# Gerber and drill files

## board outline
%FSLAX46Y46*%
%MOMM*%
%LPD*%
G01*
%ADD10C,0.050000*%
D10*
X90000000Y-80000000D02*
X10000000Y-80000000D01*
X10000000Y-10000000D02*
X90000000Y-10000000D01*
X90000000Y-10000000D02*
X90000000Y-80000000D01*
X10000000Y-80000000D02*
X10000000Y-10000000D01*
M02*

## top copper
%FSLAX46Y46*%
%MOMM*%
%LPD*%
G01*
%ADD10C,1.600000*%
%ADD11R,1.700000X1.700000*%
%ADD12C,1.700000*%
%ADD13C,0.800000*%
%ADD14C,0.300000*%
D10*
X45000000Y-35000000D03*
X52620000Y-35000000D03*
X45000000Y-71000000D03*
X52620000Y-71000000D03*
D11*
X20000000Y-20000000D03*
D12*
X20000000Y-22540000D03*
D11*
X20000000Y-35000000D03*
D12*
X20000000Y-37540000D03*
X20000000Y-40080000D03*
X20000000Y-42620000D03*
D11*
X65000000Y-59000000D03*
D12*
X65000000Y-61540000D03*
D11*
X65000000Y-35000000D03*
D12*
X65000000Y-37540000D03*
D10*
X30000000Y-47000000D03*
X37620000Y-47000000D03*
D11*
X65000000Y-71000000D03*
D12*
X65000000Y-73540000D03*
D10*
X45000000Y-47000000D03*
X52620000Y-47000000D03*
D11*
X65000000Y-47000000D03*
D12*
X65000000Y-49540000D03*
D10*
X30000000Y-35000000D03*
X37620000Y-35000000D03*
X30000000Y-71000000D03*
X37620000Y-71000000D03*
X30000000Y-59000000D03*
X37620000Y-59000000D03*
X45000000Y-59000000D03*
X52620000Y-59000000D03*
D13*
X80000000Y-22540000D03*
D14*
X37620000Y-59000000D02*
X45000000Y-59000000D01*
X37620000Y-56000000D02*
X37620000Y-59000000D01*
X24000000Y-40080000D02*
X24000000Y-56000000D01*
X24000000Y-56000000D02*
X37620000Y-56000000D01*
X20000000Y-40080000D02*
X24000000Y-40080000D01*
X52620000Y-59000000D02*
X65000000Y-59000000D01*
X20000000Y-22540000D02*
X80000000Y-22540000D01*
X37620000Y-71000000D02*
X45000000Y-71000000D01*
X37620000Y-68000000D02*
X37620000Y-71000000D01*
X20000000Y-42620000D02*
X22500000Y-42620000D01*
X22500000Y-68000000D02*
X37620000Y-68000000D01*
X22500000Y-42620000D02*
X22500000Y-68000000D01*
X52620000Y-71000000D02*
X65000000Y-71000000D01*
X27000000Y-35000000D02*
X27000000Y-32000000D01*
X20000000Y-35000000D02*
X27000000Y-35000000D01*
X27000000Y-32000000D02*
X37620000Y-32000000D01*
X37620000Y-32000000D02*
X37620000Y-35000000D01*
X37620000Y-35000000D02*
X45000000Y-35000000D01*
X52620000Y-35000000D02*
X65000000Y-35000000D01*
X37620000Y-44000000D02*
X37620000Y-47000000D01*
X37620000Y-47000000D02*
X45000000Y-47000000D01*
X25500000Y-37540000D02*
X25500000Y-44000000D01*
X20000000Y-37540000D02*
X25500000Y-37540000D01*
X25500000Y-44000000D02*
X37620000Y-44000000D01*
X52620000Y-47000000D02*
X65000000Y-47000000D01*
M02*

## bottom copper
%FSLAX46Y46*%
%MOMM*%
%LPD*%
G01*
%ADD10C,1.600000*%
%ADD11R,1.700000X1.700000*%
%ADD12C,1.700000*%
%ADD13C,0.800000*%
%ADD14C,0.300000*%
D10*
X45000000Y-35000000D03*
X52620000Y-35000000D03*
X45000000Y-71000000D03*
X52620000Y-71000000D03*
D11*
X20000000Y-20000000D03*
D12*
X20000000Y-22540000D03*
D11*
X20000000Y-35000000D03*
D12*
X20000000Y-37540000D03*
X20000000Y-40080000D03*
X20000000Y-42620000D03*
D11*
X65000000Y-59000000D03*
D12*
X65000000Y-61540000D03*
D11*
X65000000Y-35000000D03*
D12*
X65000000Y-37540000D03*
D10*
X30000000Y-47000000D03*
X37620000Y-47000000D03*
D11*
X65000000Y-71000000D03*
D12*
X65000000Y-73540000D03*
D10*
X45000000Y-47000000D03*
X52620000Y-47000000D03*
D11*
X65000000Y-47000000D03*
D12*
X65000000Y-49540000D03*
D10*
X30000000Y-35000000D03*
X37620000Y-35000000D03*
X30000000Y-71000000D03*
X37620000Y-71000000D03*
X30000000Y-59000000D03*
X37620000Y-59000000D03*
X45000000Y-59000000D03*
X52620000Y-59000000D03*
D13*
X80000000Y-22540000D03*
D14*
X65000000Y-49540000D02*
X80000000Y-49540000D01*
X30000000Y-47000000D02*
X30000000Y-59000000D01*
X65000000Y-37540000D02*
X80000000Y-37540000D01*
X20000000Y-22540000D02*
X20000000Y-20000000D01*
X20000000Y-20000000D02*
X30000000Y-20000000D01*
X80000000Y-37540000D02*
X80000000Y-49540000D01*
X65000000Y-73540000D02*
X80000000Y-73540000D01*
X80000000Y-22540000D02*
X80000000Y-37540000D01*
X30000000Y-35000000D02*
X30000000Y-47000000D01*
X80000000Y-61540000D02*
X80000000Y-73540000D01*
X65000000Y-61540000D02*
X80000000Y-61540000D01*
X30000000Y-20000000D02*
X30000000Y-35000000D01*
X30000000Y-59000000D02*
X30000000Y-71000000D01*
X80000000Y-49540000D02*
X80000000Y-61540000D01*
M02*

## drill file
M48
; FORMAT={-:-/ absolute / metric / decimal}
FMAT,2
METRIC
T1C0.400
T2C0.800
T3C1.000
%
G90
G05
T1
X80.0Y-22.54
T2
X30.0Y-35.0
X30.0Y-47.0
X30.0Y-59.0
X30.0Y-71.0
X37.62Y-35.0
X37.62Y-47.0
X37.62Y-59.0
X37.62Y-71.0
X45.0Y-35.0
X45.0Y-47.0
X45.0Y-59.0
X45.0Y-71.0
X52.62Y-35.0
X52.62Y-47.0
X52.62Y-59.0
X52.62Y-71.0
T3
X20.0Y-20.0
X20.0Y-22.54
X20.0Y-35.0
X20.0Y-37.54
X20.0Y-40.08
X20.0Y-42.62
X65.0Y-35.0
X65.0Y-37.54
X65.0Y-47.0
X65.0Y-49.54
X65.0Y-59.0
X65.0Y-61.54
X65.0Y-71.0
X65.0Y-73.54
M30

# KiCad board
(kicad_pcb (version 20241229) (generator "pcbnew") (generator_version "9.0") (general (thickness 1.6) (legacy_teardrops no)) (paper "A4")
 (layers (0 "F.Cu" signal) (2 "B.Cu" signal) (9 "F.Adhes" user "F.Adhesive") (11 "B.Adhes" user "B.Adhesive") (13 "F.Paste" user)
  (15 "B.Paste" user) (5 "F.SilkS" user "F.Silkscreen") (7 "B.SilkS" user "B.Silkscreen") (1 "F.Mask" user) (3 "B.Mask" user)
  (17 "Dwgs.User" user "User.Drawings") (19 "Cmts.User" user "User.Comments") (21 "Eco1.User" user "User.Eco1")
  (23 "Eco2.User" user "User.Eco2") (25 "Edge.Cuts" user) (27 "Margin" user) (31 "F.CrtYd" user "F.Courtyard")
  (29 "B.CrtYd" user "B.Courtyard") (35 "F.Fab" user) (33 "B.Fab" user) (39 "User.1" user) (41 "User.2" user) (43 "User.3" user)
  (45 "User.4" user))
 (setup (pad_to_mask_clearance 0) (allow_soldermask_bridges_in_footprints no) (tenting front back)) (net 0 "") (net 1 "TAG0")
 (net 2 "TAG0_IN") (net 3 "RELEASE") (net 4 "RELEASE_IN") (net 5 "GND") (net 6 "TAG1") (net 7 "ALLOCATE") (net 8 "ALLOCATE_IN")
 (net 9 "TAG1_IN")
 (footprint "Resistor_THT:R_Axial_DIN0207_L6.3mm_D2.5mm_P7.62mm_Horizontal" (layer "F.Cu") (at 45 35)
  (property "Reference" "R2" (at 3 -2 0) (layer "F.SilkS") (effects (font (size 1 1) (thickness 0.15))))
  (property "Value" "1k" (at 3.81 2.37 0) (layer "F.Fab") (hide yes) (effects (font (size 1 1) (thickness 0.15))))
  (pad "1" thru_hole circle (at 0 0) (size 1.6 1.6) (drill 0.8) (layers "*.Cu" "*.Mask") (remove_unused_layers no) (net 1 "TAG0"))
  (pad "2" thru_hole circle (at 7.62 0) (size 1.6 1.6) (drill 0.8) (layers "*.Cu" "*.Mask") (remove_unused_layers no) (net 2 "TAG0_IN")))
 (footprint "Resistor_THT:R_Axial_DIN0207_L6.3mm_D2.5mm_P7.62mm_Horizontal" (layer "F.Cu") (at 45 71)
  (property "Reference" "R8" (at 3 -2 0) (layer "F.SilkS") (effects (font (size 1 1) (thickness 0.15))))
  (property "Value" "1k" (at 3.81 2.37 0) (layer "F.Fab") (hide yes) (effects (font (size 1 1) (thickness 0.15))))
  (pad "1" thru_hole circle (at 0 0) (size 1.6 1.6) (drill 0.8) (layers "*.Cu" "*.Mask") (remove_unused_layers no) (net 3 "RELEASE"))
  (pad "2" thru_hole circle (at 7.62 0) (size 1.6 1.6) (drill 0.8) (layers "*.Cu" "*.Mask") (remove_unused_layers no) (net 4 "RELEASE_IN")))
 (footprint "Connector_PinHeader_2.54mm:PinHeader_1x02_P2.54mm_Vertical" (layer "F.Cu") (at 20 20)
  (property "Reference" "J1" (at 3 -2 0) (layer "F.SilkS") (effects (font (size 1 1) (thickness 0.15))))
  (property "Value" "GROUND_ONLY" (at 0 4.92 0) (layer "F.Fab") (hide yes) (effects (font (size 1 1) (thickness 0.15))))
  (pad "1" thru_hole rect (at 0 0) (size 1.7 1.7) (drill 1) (layers "*.Cu" "*.Mask") (remove_unused_layers no) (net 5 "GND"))
  (pad "2" thru_hole circle (at 0 2.54) (size 1.7 1.7) (drill 1) (layers "*.Cu" "*.Mask") (remove_unused_layers no) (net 5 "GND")))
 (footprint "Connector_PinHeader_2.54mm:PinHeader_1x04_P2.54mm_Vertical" (layer "F.Cu") (at 20 35)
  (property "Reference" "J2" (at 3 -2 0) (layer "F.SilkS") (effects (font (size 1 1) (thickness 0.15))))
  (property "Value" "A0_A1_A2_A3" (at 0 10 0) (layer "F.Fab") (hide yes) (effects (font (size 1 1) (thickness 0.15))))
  (pad "1" thru_hole rect (at 0 0) (size 1.7 1.7) (drill 1) (layers "*.Cu" "*.Mask") (remove_unused_layers no) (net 1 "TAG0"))
  (pad "2" thru_hole circle (at 0 2.54) (size 1.7 1.7) (drill 1) (layers "*.Cu" "*.Mask") (remove_unused_layers no) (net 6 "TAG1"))
  (pad "3" thru_hole circle (at 0 5.08) (size 1.7 1.7) (drill 1) (layers "*.Cu" "*.Mask") (remove_unused_layers no) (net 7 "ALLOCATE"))
  (pad "4" thru_hole circle (at 0 7.62) (size 1.7 1.7) (drill 1) (layers "*.Cu" "*.Mask") (remove_unused_layers no) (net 3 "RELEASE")))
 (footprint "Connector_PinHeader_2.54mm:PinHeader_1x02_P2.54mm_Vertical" (layer "F.Cu") (at 65 59)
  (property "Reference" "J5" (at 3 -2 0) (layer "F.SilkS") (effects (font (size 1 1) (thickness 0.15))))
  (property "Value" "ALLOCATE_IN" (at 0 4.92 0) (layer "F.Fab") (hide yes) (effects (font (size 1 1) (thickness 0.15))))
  (pad "1" thru_hole rect (at 0 0) (size 1.7 1.7) (drill 1) (layers "*.Cu" "*.Mask") (remove_unused_layers no) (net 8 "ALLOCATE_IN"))
  (pad "2" thru_hole circle (at 0 2.54) (size 1.7 1.7) (drill 1) (layers "*.Cu" "*.Mask") (remove_unused_layers no) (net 5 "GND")))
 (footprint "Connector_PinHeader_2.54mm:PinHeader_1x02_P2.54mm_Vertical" (layer "F.Cu") (at 65 35)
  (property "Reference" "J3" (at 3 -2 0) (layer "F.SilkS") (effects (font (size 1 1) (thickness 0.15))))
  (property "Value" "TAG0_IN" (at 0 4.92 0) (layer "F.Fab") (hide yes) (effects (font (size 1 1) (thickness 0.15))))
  (pad "1" thru_hole rect (at 0 0) (size 1.7 1.7) (drill 1) (layers "*.Cu" "*.Mask") (remove_unused_layers no) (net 2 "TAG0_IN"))
  (pad "2" thru_hole circle (at 0 2.54) (size 1.7 1.7) (drill 1) (layers "*.Cu" "*.Mask") (remove_unused_layers no) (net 5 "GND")))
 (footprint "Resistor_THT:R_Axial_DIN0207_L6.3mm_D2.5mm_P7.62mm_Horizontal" (layer "F.Cu") (at 30 47)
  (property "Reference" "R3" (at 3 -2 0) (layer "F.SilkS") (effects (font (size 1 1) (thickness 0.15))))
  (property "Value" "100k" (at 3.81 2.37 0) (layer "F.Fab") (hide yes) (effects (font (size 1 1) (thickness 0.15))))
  (pad "1" thru_hole circle (at 0 0) (size 1.6 1.6) (drill 0.8) (layers "*.Cu" "*.Mask") (remove_unused_layers no) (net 5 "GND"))
  (pad "2" thru_hole circle (at 7.62 0) (size 1.6 1.6) (drill 0.8) (layers "*.Cu" "*.Mask") (remove_unused_layers no) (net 6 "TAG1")))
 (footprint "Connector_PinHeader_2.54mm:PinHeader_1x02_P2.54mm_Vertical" (layer "F.Cu") (at 65 71)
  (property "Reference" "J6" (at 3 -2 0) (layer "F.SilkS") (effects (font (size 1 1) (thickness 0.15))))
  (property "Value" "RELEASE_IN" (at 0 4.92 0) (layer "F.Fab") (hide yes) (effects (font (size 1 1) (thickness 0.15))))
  (pad "1" thru_hole rect (at 0 0) (size 1.7 1.7) (drill 1) (layers "*.Cu" "*.Mask") (remove_unused_layers no) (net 4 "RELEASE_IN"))
  (pad "2" thru_hole circle (at 0 2.54) (size 1.7 1.7) (drill 1) (layers "*.Cu" "*.Mask") (remove_unused_layers no) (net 5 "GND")))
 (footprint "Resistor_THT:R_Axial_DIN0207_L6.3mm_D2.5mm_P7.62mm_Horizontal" (layer "F.Cu") (at 45 47)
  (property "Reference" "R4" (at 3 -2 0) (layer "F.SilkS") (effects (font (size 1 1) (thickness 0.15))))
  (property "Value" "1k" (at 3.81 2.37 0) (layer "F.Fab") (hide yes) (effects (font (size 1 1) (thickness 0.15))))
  (pad "1" thru_hole circle (at 0 0) (size 1.6 1.6) (drill 0.8) (layers "*.Cu" "*.Mask") (remove_unused_layers no) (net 6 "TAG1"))
  (pad "2" thru_hole circle (at 7.62 0) (size 1.6 1.6) (drill 0.8) (layers "*.Cu" "*.Mask") (remove_unused_layers no) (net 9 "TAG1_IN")))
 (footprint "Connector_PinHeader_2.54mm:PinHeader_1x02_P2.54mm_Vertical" (layer "F.Cu") (at 65 47)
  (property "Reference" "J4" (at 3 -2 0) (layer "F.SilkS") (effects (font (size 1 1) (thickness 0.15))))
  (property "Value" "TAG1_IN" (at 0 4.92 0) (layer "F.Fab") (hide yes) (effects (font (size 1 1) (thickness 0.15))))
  (pad "1" thru_hole rect (at 0 0) (size 1.7 1.7) (drill 1) (layers "*.Cu" "*.Mask") (remove_unused_layers no) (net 9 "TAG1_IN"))
  (pad "2" thru_hole circle (at 0 2.54) (size 1.7 1.7) (drill 1) (layers "*.Cu" "*.Mask") (remove_unused_layers no) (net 5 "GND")))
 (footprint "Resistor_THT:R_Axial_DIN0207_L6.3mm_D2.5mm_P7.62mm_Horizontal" (layer "F.Cu") (at 30 35)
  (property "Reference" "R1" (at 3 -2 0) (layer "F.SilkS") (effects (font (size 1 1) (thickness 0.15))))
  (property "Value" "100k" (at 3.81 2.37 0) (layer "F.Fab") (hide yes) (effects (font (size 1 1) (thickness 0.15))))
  (pad "1" thru_hole circle (at 0 0) (size 1.6 1.6) (drill 0.8) (layers "*.Cu" "*.Mask") (remove_unused_layers no) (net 5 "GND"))
  (pad "2" thru_hole circle (at 7.62 0) (size 1.6 1.6) (drill 0.8) (layers "*.Cu" "*.Mask") (remove_unused_layers no) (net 1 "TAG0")))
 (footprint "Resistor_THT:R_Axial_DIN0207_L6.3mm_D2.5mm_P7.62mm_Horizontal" (layer "F.Cu") (at 30 71)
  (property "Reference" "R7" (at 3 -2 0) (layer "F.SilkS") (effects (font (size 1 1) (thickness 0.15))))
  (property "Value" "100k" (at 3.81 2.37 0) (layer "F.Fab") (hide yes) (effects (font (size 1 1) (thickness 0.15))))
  (pad "1" thru_hole circle (at 0 0) (size 1.6 1.6) (drill 0.8) (layers "*.Cu" "*.Mask") (remove_unused_layers no) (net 5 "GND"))
  (pad "2" thru_hole circle (at 7.62 0) (size 1.6 1.6) (drill 0.8) (layers "*.Cu" "*.Mask") (remove_unused_layers no) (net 3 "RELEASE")))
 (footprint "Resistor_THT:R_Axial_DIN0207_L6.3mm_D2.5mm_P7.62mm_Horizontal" (layer "F.Cu") (at 30 59)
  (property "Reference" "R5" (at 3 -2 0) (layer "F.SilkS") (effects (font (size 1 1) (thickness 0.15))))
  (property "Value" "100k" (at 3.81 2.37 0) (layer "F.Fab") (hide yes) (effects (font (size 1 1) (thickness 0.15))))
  (pad "1" thru_hole circle (at 0 0) (size 1.6 1.6) (drill 0.8) (layers "*.Cu" "*.Mask") (remove_unused_layers no) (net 5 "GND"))
  (pad "2" thru_hole circle (at 7.62 0) (size 1.6 1.6) (drill 0.8) (layers "*.Cu" "*.Mask") (remove_unused_layers no) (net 7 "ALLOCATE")))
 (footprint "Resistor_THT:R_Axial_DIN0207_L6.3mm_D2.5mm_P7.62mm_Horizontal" (layer "F.Cu") (at 45 59)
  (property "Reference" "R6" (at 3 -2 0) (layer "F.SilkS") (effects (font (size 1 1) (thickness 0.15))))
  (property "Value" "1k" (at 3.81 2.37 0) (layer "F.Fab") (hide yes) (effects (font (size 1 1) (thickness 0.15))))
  (pad "1" thru_hole circle (at 0 0) (size 1.6 1.6) (drill 0.8) (layers "*.Cu" "*.Mask") (remove_unused_layers no) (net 7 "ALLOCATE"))
  (pad "2" thru_hole circle (at 7.62 0) (size 1.6 1.6) (drill 0.8) (layers "*.Cu" "*.Mask") (remove_unused_layers no) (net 8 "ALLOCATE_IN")))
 (gr_line (start 90 80) (end 10 80) (stroke (width 0.05) (type default)) (layer "Edge.Cuts"))
 (gr_line (start 10 10) (end 90 10) (stroke (width 0.05) (type default)) (layer "Edge.Cuts"))
 (gr_line (start 90 10) (end 90 80) (stroke (width 0.05) (type default)) (layer "Edge.Cuts"))
 (gr_line (start 10 80) (end 10 10) (stroke (width 0.05) (type default)) (layer "Edge.Cuts"))
 (segment (start 37.62 59) (end 45 59) (width 0.3) (layer "F.Cu") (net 7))
 (segment (start 37.62 56) (end 37.62 59) (width 0.3) (layer "F.Cu") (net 7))
 (segment (start 24 40.08) (end 24 56) (width 0.3) (layer "F.Cu") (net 7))
 (segment (start 24 56) (end 37.62 56) (width 0.3) (layer "F.Cu") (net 7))
 (segment (start 20 40.08) (end 24 40.08) (width 0.3) (layer "F.Cu") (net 7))
 (segment (start 52.62 59) (end 65 59) (width 0.3) (layer "F.Cu") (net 8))
 (segment (start 20 22.54) (end 80 22.54) (width 0.3) (layer "F.Cu") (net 5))
 (via (at 80 22.54) (size 0.8) (drill 0.4) (layers "F.Cu" "B.Cu") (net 5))
 (segment (start 65 49.54) (end 80 49.54) (width 0.3) (layer "B.Cu") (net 5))
 (segment (start 30 47) (end 30 59) (width 0.3) (layer "B.Cu") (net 5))
 (segment (start 65 37.54) (end 80 37.54) (width 0.3) (layer "B.Cu") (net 5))
 (segment (start 20 22.54) (end 20 20) (width 0.3) (layer "B.Cu") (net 5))
 (segment (start 20 20) (end 30 20) (width 0.3) (layer "B.Cu") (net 5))
 (segment (start 80 37.54) (end 80 49.54) (width 0.3) (layer "B.Cu") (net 5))
 (segment (start 65 73.54) (end 80 73.54) (width 0.3) (layer "B.Cu") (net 5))
 (segment (start 80 22.54) (end 80 37.54) (width 0.3) (layer "B.Cu") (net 5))
 (segment (start 30 35) (end 30 47) (width 0.3) (layer "B.Cu") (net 5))
 (segment (start 80 61.54) (end 80 73.54) (width 0.3) (layer "B.Cu") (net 5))
 (segment (start 65 61.54) (end 80 61.54) (width 0.3) (layer "B.Cu") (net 5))
 (segment (start 30 20) (end 30 35) (width 0.3) (layer "B.Cu") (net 5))
 (segment (start 30 59) (end 30 71) (width 0.3) (layer "B.Cu") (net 5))
 (segment (start 80 49.54) (end 80 61.54) (width 0.3) (layer "B.Cu") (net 5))
 (segment (start 37.62 71) (end 45 71) (width 0.3) (layer "F.Cu") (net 3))
 (segment (start 37.62 68) (end 37.62 71) (width 0.3) (layer "F.Cu") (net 3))
 (segment (start 20 42.62) (end 22.5 42.62) (width 0.3) (layer "F.Cu") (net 3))
 (segment (start 22.5 68) (end 37.62 68) (width 0.3) (layer "F.Cu") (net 3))
 (segment (start 22.5 42.62) (end 22.5 68) (width 0.3) (layer "F.Cu") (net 3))
 (segment (start 52.62 71) (end 65 71) (width 0.3) (layer "F.Cu") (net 4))
 (segment (start 27 35) (end 27 32) (width 0.3) (layer "F.Cu") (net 1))
 (segment (start 20 35) (end 27 35) (width 0.3) (layer "F.Cu") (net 1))
 (segment (start 27 32) (end 37.62 32) (width 0.3) (layer "F.Cu") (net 1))
 (segment (start 37.62 32) (end 37.62 35) (width 0.3) (layer "F.Cu") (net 1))
 (segment (start 37.62 35) (end 45 35) (width 0.3) (layer "F.Cu") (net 1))
 (segment (start 52.62 35) (end 65 35) (width 0.3) (layer "F.Cu") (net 2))
 (segment (start 37.62 44) (end 37.62 47) (width 0.3) (layer "F.Cu") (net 6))
 (segment (start 37.62 47) (end 45 47) (width 0.3) (layer "F.Cu") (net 6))
 (segment (start 25.5 37.54) (end 25.5 44) (width 0.3) (layer "F.Cu") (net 6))
 (segment (start 20 37.54) (end 25.5 37.54) (width 0.3) (layer "F.Cu") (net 6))
 (segment (start 25.5 44) (end 37.62 44) (width 0.3) (layer "F.Cu") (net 6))
 (segment (start 52.62 47) (end 65 47) (width 0.3) (layer "F.Cu") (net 9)))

